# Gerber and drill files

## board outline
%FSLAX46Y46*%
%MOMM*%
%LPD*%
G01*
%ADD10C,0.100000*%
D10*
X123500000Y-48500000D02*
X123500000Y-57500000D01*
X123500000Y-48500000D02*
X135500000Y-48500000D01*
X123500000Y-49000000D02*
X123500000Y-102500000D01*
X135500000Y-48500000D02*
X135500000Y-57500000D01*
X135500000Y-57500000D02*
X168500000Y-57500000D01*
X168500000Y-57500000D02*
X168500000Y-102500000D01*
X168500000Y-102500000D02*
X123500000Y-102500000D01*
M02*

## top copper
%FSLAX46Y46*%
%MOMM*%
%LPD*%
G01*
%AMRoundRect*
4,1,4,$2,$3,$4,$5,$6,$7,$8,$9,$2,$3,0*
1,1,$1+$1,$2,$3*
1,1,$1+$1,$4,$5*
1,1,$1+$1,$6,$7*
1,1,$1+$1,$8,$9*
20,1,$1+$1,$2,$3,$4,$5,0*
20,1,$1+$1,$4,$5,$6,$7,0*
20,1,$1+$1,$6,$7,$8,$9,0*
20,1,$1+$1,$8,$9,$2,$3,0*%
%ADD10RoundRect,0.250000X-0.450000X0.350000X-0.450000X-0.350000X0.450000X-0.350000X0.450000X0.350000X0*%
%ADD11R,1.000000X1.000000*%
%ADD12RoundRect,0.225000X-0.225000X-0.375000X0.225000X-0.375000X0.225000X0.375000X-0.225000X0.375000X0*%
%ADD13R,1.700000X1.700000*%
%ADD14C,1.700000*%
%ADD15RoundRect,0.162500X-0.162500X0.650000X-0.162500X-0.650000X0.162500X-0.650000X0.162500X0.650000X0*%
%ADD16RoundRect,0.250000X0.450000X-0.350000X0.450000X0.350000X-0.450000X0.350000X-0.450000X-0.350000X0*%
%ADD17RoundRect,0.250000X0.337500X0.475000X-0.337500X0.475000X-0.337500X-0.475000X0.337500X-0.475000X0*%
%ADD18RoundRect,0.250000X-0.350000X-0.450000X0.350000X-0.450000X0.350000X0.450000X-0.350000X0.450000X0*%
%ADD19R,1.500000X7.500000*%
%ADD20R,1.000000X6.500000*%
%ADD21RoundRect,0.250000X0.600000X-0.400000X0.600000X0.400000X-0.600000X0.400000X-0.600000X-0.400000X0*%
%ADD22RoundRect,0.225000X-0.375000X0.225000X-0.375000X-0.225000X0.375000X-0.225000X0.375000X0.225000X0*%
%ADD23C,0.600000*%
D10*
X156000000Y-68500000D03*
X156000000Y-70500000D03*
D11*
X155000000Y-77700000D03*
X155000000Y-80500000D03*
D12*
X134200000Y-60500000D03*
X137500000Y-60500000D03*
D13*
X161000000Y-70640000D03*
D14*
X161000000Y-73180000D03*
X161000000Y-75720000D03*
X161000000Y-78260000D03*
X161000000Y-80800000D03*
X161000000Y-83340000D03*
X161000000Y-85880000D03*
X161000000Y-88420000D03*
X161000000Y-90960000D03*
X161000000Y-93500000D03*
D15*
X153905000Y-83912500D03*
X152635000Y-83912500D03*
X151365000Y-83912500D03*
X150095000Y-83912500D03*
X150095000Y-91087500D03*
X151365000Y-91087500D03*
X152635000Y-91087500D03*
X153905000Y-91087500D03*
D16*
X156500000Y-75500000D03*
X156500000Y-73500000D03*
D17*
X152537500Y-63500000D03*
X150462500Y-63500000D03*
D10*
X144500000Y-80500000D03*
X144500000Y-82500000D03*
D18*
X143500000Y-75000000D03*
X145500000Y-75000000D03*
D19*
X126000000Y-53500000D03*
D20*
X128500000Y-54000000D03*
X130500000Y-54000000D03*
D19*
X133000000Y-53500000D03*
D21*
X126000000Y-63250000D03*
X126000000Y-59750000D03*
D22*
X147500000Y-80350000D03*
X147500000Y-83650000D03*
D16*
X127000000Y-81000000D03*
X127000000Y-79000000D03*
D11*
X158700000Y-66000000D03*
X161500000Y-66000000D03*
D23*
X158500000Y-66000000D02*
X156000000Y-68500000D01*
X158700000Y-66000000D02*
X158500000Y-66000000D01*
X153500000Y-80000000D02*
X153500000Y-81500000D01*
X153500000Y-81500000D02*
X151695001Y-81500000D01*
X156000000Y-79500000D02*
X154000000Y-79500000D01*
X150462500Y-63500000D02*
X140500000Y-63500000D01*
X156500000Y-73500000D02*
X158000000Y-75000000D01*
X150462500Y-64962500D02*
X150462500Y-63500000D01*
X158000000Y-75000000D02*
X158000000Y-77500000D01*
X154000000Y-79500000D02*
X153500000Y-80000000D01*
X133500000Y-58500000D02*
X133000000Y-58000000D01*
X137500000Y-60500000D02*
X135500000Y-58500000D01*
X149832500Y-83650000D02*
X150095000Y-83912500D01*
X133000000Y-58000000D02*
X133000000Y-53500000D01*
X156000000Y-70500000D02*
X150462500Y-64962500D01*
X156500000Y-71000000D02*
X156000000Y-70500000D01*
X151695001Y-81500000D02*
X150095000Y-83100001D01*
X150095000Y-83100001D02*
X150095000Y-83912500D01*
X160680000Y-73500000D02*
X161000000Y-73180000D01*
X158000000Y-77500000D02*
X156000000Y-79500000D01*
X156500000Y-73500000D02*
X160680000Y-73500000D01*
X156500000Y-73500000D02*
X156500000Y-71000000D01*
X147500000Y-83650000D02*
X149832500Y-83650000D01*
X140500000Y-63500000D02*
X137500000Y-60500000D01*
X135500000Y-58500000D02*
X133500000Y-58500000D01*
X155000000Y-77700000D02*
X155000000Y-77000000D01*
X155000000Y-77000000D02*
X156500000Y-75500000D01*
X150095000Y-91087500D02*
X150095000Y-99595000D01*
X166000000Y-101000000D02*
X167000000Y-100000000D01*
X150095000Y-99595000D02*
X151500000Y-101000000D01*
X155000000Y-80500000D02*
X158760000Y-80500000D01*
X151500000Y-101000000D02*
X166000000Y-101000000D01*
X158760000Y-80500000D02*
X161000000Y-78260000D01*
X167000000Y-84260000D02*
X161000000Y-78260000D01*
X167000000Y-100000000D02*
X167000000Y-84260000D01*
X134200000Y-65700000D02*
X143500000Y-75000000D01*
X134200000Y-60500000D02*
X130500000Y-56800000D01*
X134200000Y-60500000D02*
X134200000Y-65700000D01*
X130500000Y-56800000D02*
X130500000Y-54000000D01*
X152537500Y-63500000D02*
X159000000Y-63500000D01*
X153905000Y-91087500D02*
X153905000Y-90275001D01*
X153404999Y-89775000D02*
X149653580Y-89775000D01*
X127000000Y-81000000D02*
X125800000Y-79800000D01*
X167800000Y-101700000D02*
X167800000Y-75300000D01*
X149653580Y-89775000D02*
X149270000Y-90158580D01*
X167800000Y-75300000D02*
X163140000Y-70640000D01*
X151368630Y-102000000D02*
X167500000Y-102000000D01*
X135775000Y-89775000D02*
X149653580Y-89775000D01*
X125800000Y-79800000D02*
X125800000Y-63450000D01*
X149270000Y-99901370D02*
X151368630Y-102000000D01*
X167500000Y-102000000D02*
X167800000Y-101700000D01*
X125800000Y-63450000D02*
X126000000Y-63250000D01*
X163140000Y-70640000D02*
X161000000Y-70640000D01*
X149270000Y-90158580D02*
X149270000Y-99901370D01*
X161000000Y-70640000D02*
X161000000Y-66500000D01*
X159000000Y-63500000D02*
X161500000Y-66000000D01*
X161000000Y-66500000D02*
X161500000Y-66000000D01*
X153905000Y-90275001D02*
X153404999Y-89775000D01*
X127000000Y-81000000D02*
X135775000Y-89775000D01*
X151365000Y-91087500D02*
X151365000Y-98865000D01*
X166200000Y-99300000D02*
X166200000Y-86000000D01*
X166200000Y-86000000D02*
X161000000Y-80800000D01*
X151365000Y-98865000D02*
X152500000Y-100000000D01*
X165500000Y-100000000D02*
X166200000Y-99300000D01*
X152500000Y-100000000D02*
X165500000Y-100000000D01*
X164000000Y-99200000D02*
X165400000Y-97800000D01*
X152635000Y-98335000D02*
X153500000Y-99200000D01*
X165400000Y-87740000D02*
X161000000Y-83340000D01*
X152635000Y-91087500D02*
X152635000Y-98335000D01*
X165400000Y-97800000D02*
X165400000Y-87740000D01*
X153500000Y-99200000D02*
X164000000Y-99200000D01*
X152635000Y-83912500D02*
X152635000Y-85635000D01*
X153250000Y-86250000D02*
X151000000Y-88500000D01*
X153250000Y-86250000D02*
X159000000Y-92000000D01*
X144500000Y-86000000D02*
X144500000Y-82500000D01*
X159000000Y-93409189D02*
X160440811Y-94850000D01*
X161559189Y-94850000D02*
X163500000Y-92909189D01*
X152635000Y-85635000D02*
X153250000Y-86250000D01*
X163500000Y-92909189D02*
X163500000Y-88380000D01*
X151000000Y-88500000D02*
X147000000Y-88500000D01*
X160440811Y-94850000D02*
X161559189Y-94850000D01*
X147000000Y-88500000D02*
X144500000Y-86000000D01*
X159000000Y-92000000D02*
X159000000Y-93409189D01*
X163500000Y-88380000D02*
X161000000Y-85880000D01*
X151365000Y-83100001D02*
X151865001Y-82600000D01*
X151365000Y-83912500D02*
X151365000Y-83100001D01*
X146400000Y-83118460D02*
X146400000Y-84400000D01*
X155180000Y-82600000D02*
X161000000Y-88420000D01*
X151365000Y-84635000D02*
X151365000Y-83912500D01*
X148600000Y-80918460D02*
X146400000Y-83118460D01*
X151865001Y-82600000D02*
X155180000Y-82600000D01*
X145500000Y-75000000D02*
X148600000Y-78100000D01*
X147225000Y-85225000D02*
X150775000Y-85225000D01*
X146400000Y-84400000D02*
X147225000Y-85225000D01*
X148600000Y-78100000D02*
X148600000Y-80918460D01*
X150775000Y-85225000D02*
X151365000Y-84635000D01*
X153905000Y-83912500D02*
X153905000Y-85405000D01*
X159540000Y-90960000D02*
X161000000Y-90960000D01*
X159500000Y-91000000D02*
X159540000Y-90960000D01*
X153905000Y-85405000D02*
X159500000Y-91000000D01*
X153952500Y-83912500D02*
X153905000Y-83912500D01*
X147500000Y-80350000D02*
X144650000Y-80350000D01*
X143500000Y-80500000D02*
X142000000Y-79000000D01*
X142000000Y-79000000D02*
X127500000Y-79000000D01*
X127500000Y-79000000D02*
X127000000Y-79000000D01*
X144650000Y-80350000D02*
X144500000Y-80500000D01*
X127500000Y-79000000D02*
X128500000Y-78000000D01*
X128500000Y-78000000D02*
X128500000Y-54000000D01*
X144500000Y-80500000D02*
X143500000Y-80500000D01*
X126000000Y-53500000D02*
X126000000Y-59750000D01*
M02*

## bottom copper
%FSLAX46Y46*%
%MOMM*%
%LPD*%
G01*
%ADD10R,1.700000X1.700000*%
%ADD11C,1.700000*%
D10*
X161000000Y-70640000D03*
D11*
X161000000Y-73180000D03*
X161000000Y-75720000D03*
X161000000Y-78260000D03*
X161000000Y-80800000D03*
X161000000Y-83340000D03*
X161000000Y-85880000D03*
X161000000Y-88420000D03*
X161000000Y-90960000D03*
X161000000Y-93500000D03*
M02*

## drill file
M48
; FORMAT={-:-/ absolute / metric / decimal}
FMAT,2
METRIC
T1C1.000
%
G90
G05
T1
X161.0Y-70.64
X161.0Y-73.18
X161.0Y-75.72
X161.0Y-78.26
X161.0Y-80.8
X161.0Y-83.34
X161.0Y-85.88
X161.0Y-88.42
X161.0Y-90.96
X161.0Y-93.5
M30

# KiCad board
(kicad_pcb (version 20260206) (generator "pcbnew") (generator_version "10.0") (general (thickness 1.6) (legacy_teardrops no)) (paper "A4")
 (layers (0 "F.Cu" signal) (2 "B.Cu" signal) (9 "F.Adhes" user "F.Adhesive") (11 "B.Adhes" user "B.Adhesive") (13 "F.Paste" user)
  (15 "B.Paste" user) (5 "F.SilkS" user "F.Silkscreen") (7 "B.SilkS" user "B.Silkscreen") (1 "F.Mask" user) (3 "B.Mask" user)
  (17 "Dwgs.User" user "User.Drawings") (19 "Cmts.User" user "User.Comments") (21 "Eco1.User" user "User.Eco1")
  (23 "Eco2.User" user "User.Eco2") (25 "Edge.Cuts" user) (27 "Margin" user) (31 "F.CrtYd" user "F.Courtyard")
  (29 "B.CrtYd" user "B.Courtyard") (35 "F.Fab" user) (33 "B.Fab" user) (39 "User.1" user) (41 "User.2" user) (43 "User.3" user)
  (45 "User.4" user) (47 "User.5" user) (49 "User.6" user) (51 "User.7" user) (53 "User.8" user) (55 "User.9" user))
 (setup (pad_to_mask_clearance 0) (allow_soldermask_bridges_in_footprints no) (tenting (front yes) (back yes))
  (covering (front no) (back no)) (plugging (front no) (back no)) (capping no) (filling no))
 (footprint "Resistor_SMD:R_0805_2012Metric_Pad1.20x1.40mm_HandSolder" (layer "F.Cu") (at 156 69.5 -90)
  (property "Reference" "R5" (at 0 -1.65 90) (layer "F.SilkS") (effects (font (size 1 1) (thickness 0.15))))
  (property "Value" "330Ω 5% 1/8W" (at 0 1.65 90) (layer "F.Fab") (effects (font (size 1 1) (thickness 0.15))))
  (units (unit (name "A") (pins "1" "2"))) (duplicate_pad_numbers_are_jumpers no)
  (pad "1" smd roundrect (at -1 0 270) (size 1.2 1.4) (layers "F.Cu" "F.Mask" "F.Paste") (roundrect_rratio 0.208333) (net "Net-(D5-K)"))
  (pad "2" smd roundrect (at 1 0 270) (size 1.2 1.4) (layers "F.Cu" "F.Mask" "F.Paste") (roundrect_rratio 0.208333) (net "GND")))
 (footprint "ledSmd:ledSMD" (layer "F.Cu") (at 155 79.5 -90)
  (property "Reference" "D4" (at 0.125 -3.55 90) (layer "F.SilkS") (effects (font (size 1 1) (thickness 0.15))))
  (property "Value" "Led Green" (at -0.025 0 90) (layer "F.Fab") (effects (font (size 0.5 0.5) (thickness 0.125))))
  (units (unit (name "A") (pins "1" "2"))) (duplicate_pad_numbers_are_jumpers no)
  (pad "1" smd rect (at -1.8 0 270) (size 1 1) (layers "F.Cu" "F.Mask" "F.Paste") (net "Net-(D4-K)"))
  (pad "2" smd rect (at 1 0 270) (size 1 1) (layers "F.Cu" "F.Mask" "F.Paste") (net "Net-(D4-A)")))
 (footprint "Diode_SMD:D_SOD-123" (layer "F.Cu") (at 135.85 60.5)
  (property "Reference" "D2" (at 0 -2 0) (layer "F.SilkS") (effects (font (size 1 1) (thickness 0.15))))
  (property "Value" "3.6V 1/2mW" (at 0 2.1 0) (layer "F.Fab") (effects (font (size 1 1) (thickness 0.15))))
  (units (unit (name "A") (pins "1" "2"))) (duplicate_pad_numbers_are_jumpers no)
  (pad "1" smd roundrect (at -1.65 0) (size 0.9 1.2) (layers "F.Cu" "F.Mask" "F.Paste") (roundrect_rratio 0.25) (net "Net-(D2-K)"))
  (pad "2" smd roundrect (at 1.65 0) (size 0.9 1.2) (layers "F.Cu" "F.Mask" "F.Paste") (roundrect_rratio 0.25) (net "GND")))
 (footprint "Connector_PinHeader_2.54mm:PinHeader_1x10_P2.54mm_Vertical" (layer "F.Cu") (at 161 70.64)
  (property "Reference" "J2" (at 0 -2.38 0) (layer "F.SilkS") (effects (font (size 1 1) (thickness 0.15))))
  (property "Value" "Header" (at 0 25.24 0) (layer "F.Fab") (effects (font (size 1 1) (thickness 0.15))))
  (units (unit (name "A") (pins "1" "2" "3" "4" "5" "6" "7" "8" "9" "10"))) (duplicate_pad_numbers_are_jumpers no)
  (pad "1" thru_hole rect (at 0 0) (size 1.7 1.7) (drill 1) (layers "*.Cu" "*.Mask") (remove_unused_layers no) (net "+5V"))
  (pad "2" thru_hole circle (at 0 2.54) (size 1.7 1.7) (drill 1) (layers "*.Cu" "*.Mask") (remove_unused_layers no) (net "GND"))
  (pad "3" thru_hole circle (at 0 5.08) (size 1.7 1.7) (drill 1) (layers "*.Cu" "*.Mask") (remove_unused_layers no)
   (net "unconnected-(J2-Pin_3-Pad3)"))
  (pad "4" thru_hole circle (at 0 7.62) (size 1.7 1.7) (drill 1) (layers "*.Cu" "*.Mask") (remove_unused_layers no) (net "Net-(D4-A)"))
  (pad "5" thru_hole circle (at 0 10.16) (size 1.7 1.7) (drill 1) (layers "*.Cu" "*.Mask") (remove_unused_layers no) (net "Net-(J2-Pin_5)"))
  (pad "6" thru_hole circle (at 0 12.7) (size 1.7 1.7) (drill 1) (layers "*.Cu" "*.Mask") (remove_unused_layers no) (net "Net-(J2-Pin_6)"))
  (pad "7" thru_hole circle (at 0 15.24) (size 1.7 1.7) (drill 1) (layers "*.Cu" "*.Mask") (remove_unused_layers no) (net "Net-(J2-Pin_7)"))
  (pad "8" thru_hole circle (at 0 17.78) (size 1.7 1.7) (drill 1) (layers "*.Cu" "*.Mask") (remove_unused_layers no) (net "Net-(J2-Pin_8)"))
  (pad "9" thru_hole circle (at 0 20.32) (size 1.7 1.7) (drill 1) (layers "*.Cu" "*.Mask") (remove_unused_layers no) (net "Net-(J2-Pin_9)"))
  (pad "10" thru_hole circle (at 0 22.86) (size 1.7 1.7) (drill 1) (layers "*.Cu" "*.Mask") (remove_unused_layers no)
   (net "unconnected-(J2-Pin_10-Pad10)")))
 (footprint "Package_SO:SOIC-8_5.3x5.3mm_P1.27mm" (layer "F.Cu") (at 152 87.5 -90)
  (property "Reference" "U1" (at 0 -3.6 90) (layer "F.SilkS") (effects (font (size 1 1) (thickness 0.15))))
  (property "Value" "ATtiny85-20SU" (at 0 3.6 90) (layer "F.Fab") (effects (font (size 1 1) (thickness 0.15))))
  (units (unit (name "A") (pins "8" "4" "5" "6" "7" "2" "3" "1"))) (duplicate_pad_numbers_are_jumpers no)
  (pad "1" smd roundrect (at -3.5875 -1.905 270) (size 1.625 0.65) (layers "F.Cu" "F.Mask" "F.Paste") (roundrect_rratio 0.25)
   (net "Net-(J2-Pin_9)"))
  (pad "2" smd roundrect (at -3.5875 -0.635 270) (size 1.625 0.65) (layers "F.Cu" "F.Mask" "F.Paste") (roundrect_rratio 0.25)
   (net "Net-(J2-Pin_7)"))
  (pad "3" smd roundrect (at -3.5875 0.635 270) (size 1.625 0.65) (layers "F.Cu" "F.Mask" "F.Paste") (roundrect_rratio 0.25)
   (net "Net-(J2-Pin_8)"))
  (pad "4" smd roundrect (at -3.5875 1.905 270) (size 1.625 0.65) (layers "F.Cu" "F.Mask" "F.Paste") (roundrect_rratio 0.25) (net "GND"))
  (pad "5" smd roundrect (at 3.5875 1.905 270) (size 1.625 0.65) (layers "F.Cu" "F.Mask" "F.Paste") (roundrect_rratio 0.25)
   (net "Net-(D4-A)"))
  (pad "6" smd roundrect (at 3.5875 0.635 270) (size 1.625 0.65) (layers "F.Cu" "F.Mask" "F.Paste") (roundrect_rratio 0.25)
   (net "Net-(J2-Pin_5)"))
  (pad "7" smd roundrect (at 3.5875 -0.635 270) (size 1.625 0.65) (layers "F.Cu" "F.Mask" "F.Paste") (roundrect_rratio 0.25)
   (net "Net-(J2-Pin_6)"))
  (pad "8" smd roundrect (at 3.5875 -1.905 270) (size 1.625 0.65) (layers "F.Cu" "F.Mask" "F.Paste") (roundrect_rratio 0.25) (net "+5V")))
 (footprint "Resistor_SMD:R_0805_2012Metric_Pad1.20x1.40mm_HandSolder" (layer "F.Cu") (at 156.5 74.5 90)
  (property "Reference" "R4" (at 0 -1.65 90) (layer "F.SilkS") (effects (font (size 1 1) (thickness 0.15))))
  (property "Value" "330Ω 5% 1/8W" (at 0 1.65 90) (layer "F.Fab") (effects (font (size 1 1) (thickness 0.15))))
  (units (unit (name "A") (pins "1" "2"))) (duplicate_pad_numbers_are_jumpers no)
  (pad "1" smd roundrect (at -1 0 90) (size 1.2 1.4) (layers "F.Cu" "F.Mask" "F.Paste") (roundrect_rratio 0.208333) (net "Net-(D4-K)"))
  (pad "2" smd roundrect (at 1 0 90) (size 1.2 1.4) (layers "F.Cu" "F.Mask" "F.Paste") (roundrect_rratio 0.208333) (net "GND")))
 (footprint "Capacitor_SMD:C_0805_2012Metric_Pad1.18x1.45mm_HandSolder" (layer "F.Cu") (at 151.5 63.5 180)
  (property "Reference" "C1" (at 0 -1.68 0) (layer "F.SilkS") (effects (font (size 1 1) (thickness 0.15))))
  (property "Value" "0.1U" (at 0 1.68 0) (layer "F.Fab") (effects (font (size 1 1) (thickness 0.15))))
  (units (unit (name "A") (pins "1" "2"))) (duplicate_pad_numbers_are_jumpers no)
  (pad "1" smd roundrect (at -1.0375 0 180) (size 1.175 1.45) (layers "F.Cu" "F.Mask" "F.Paste") (roundrect_rratio 0.212766) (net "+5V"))
  (pad "2" smd roundrect (at 1.0375 0 180) (size 1.175 1.45) (layers "F.Cu" "F.Mask" "F.Paste") (roundrect_rratio 0.212766) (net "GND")))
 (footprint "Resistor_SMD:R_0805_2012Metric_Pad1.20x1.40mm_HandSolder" (layer "F.Cu") (at 144.5 81.5 -90)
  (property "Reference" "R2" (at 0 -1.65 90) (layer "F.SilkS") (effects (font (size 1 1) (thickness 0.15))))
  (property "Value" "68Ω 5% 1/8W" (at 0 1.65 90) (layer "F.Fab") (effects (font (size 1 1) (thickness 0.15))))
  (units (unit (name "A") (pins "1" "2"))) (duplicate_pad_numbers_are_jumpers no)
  (pad "1" smd roundrect (at -1 0 270) (size 1.2 1.4) (layers "F.Cu" "F.Mask" "F.Paste") (roundrect_rratio 0.208333) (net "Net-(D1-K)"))
  (pad "2" smd roundrect (at 1 0 270) (size 1.2 1.4) (layers "F.Cu" "F.Mask" "F.Paste") (roundrect_rratio 0.208333) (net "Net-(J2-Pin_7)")))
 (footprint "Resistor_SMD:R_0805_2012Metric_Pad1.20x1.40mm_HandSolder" (layer "F.Cu") (at 144.5 75)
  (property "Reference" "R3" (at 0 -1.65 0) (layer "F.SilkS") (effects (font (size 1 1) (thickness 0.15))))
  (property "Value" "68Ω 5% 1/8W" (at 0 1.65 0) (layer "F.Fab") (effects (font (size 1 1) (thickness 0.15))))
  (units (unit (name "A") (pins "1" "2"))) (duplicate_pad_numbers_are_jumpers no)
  (pad "1" smd roundrect (at -1 0) (size 1.2 1.4) (layers "F.Cu" "F.Mask" "F.Paste") (roundrect_rratio 0.208333) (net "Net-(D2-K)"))
  (pad "2" smd roundrect (at 1 0) (size 1.2 1.4) (layers "F.Cu" "F.Mask" "F.Paste") (roundrect_rratio 0.208333) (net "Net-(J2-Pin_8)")))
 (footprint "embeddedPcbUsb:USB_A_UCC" (layer "F.Cu") (at 129.5 53.7 -90)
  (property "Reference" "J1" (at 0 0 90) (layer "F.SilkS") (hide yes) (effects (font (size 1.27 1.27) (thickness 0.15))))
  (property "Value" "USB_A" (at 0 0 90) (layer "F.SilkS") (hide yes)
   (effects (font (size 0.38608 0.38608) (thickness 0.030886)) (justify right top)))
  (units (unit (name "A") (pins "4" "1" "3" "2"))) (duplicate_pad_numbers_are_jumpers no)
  (pad "1" smd rect (at -0.2 3.5 270) (size 7.5 1.5) (layers "F.Cu" "F.Mask" "F.Paste") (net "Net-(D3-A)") (solder_mask_margin 0.1016))
  (pad "2" smd rect (at 0.3 1 270) (size 6.5 1) (layers "F.Cu" "F.Mask" "F.Paste") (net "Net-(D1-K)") (solder_mask_margin 0.1016))
  (pad "3" smd rect (at 0.3 -1 270) (size 6.5 1) (layers "F.Cu" "F.Mask" "F.Paste") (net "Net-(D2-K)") (solder_mask_margin 0.1016))
  (pad "4" smd rect (at -0.2 -3.5 270) (size 7.5 1.5) (layers "F.Cu" "F.Mask" "F.Paste") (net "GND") (solder_mask_margin 0.1016)))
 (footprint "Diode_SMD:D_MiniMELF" (layer "F.Cu") (at 126 61.5 90)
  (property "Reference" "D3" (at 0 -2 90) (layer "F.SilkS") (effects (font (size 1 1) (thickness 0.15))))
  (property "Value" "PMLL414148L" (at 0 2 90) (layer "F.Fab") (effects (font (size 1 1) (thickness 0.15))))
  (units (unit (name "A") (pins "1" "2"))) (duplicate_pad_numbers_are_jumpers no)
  (pad "1" smd roundrect (at -1.75 0 90) (size 1.3 1.7) (layers "F.Cu" "F.Mask" "F.Paste") (roundrect_rratio 0.1923076923) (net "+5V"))
  (pad "2" smd roundrect (at 1.75 0 90) (size 1.3 1.7) (layers "F.Cu" "F.Mask" "F.Paste") (roundrect_rratio 0.1923076923) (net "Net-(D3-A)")))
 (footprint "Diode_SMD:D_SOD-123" (layer "F.Cu") (at 147.5 82 -90)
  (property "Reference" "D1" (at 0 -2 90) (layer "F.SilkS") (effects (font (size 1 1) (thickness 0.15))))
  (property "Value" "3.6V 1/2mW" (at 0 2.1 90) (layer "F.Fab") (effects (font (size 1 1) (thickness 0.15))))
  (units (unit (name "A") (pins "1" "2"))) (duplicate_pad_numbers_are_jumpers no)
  (pad "1" smd roundrect (at -1.65 0 270) (size 0.9 1.2) (layers "F.Cu" "F.Mask" "F.Paste") (roundrect_rratio 0.25) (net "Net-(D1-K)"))
  (pad "2" smd roundrect (at 1.65 0 270) (size 0.9 1.2) (layers "F.Cu" "F.Mask" "F.Paste") (roundrect_rratio 0.25) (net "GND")))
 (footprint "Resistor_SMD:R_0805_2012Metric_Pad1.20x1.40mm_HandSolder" (layer "F.Cu") (at 127 80 90)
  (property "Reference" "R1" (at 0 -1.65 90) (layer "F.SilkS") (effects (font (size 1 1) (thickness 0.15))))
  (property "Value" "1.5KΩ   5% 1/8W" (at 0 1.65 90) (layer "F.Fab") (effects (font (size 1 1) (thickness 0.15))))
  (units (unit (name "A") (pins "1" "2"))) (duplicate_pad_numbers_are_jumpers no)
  (pad "1" smd roundrect (at -1 0 90) (size 1.2 1.4) (layers "F.Cu" "F.Mask" "F.Paste") (roundrect_rratio 0.208333) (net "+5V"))
  (pad "2" smd roundrect (at 1 0 90) (size 1.2 1.4) (layers "F.Cu" "F.Mask" "F.Paste") (roundrect_rratio 0.208333) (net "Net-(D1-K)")))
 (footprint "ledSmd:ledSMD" (layer "F.Cu") (at 160.5 66)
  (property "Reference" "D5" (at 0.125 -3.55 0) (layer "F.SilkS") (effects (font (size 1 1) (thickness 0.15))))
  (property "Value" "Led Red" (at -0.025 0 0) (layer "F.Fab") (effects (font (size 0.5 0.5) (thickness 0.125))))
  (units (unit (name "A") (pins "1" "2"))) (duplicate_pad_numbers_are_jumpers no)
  (pad "1" smd rect (at -1.8 0) (size 1 1) (layers "F.Cu" "F.Mask" "F.Paste") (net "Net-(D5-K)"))
  (pad "2" smd rect (at 1 0) (size 1 1) (layers "F.Cu" "F.Mask" "F.Paste") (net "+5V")))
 (gr_line (start 123.5 48.5) (end 123.5 57.5) (stroke (width 0.1) (type default)) (layer "Edge.Cuts"))
 (gr_line (start 123.5 48.5) (end 135.5 48.5) (stroke (width 0.1) (type default)) (layer "Edge.Cuts"))
 (gr_line (start 123.5 49) (end 123.5 102.5) (stroke (width 0.1) (type default)) (layer "Edge.Cuts"))
 (gr_line (start 135.5 48.5) (end 135.5 57.5) (stroke (width 0.1) (type default)) (layer "Edge.Cuts"))
 (gr_line (start 135.5 57.5) (end 168.5 57.5) (stroke (width 0.1) (type default)) (layer "Edge.Cuts"))
 (gr_line (start 168.5 57.5) (end 168.5 102.5) (stroke (width 0.1) (type default)) (layer "Edge.Cuts"))
 (gr_line (start 168.5 102.5) (end 123.5 102.5) (stroke (width 0.1) (type default)) (layer "Edge.Cuts"))
 (segment (start 158.5 66) (end 156 68.5) (width 0.6) (layer "F.Cu") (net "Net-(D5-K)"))
 (segment (start 158.7 66) (end 158.5 66) (width 0.6) (layer "F.Cu") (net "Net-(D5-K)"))
 (segment (start 153.5 80) (end 153.5 81.5) (width 0.6) (layer "F.Cu") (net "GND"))
 (segment (start 153.5 81.5) (end 151.695001 81.5) (width 0.6) (layer "F.Cu") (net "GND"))
 (segment (start 156 79.5) (end 154 79.5) (width 0.6) (layer "F.Cu") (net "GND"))
 (segment (start 150.4625 63.5) (end 140.5 63.5) (width 0.6) (layer "F.Cu") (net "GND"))
 (segment (start 156.5 73.5) (end 158 75) (width 0.6) (layer "F.Cu") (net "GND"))
 (segment (start 150.4625 64.9625) (end 150.4625 63.5) (width 0.6) (layer "F.Cu") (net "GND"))
 (segment (start 158 75) (end 158 77.5) (width 0.6) (layer "F.Cu") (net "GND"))
 (segment (start 154 79.5) (end 153.5 80) (width 0.6) (layer "F.Cu") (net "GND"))
 (segment (start 133.5 58.5) (end 133 58) (width 0.6) (layer "F.Cu") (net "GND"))
 (segment (start 137.5 60.5) (end 135.5 58.5) (width 0.6) (layer "F.Cu") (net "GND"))
 (segment (start 149.8325 83.65) (end 150.095 83.9125) (width 0.6) (layer "F.Cu") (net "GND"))
 (segment (start 133 58) (end 133 53.5) (width 0.6) (layer "F.Cu") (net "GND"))
 (segment (start 156 70.5) (end 150.4625 64.9625) (width 0.6) (layer "F.Cu") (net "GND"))
 (segment (start 156.5 71) (end 156 70.5) (width 0.6) (layer "F.Cu") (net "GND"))
 (segment (start 151.695001 81.5) (end 150.095 83.100001) (width 0.6) (layer "F.Cu") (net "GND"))
 (segment (start 150.095 83.100001) (end 150.095 83.9125) (width 0.6) (layer "F.Cu") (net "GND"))
 (segment (start 160.68 73.5) (end 161 73.18) (width 0.6) (layer "F.Cu") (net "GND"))
 (segment (start 158 77.5) (end 156 79.5) (width 0.6) (layer "F.Cu") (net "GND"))
 (segment (start 156.5 73.5) (end 160.68 73.5) (width 0.6) (layer "F.Cu") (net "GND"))
 (segment (start 156.5 73.5) (end 156.5 71) (width 0.6) (layer "F.Cu") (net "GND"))
 (segment (start 147.5 83.65) (end 149.8325 83.65) (width 0.6) (layer "F.Cu") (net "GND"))
 (segment (start 140.5 63.5) (end 137.5 60.5) (width 0.6) (layer "F.Cu") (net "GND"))
 (segment (start 135.5 58.5) (end 133.5 58.5) (width 0.6) (layer "F.Cu") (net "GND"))
 (segment (start 155 77.7) (end 155 77) (width 0.6) (layer "F.Cu") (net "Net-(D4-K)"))
 (segment (start 155 77) (end 156.5 75.5) (width 0.6) (layer "F.Cu") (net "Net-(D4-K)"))
 (segment (start 150.095 91.0875) (end 150.095 99.595) (width 0.6) (layer "F.Cu") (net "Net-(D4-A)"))
 (segment (start 166 101) (end 167 100) (width 0.6) (layer "F.Cu") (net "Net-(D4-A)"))
 (segment (start 150.095 99.595) (end 151.5 101) (width 0.6) (layer "F.Cu") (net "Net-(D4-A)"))
 (segment (start 155 80.5) (end 158.76 80.5) (width 0.6) (layer "F.Cu") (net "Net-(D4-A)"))
 (segment (start 151.5 101) (end 166 101) (width 0.6) (layer "F.Cu") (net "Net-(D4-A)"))
 (segment (start 158.76 80.5) (end 161 78.26) (width 0.6) (layer "F.Cu") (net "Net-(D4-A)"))
 (segment (start 167 84.26) (end 161 78.26) (width 0.6) (layer "F.Cu") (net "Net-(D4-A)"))
 (segment (start 167 100) (end 167 84.26) (width 0.6) (layer "F.Cu") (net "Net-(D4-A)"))
 (segment (start 134.2 65.7) (end 143.5 75) (width 0.6) (layer "F.Cu") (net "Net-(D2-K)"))
 (segment (start 134.2 60.5) (end 130.5 56.8) (width 0.6) (layer "F.Cu") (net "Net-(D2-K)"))
 (segment (start 134.2 60.5) (end 134.2 65.7) (width 0.6) (layer "F.Cu") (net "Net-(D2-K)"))
 (segment (start 130.5 56.8) (end 130.5 54) (width 0.6) (layer "F.Cu") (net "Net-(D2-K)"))
 (segment (start 152.5375 63.5) (end 159 63.5) (width 0.6) (layer "F.Cu") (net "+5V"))
 (segment (start 153.905 91.0875) (end 153.905 90.275001) (width 0.6) (layer "F.Cu") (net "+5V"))
 (segment (start 153.404999 89.775) (end 149.65358 89.775) (width 0.6) (layer "F.Cu") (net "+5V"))
 (segment (start 127 81) (end 125.8 79.8) (width 0.6) (layer "F.Cu") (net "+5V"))
 (segment (start 167.8 101.7) (end 167.8 75.3) (width 0.6) (layer "F.Cu") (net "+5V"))
 (segment (start 149.65358 89.775) (end 149.27 90.15858) (width 0.6) (layer "F.Cu") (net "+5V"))
 (segment (start 167.8 75.3) (end 163.14 70.64) (width 0.6) (layer "F.Cu") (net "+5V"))
 (segment (start 151.36863 102) (end 167.5 102) (width 0.6) (layer "F.Cu") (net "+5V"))
 (segment (start 135.775 89.775) (end 149.65358 89.775) (width 0.6) (layer "F.Cu") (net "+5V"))
 (segment (start 125.8 79.8) (end 125.8 63.45) (width 0.6) (layer "F.Cu") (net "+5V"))
 (segment (start 149.27 99.90137) (end 151.36863 102) (width 0.6) (layer "F.Cu") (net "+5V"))
 (segment (start 167.5 102) (end 167.8 101.7) (width 0.6) (layer "F.Cu") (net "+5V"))
 (segment (start 125.8 63.45) (end 126 63.25) (width 0.6) (layer "F.Cu") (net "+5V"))
 (segment (start 163.14 70.64) (end 161 70.64) (width 0.6) (layer "F.Cu") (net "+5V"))
 (segment (start 149.27 90.15858) (end 149.27 99.90137) (width 0.6) (layer "F.Cu") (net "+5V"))
 (segment (start 161 70.64) (end 161 66.5) (width 0.6) (layer "F.Cu") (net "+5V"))
 (segment (start 159 63.5) (end 161.5 66) (width 0.6) (layer "F.Cu") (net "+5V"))
 (segment (start 161 66.5) (end 161.5 66) (width 0.6) (layer "F.Cu") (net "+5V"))
 (segment (start 153.905 90.275001) (end 153.404999 89.775) (width 0.6) (layer "F.Cu") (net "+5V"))
 (segment (start 127 81) (end 135.775 89.775) (width 0.6) (layer "F.Cu") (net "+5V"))
 (segment (start 151.365 91.0875) (end 151.365 98.865) (width 0.6) (layer "F.Cu") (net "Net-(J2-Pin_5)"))
 (segment (start 166.2 99.3) (end 166.2 86) (width 0.6) (layer "F.Cu") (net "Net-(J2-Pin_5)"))
 (segment (start 166.2 86) (end 161 80.8) (width 0.6) (layer "F.Cu") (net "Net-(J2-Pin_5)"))
 (segment (start 151.365 98.865) (end 152.5 100) (width 0.6) (layer "F.Cu") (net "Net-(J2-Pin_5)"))
 (segment (start 165.5 100) (end 166.2 99.3) (width 0.6) (layer "F.Cu") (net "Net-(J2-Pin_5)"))
 (segment (start 152.5 100) (end 165.5 100) (width 0.6) (layer "F.Cu") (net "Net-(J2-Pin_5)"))
 (segment (start 164 99.2) (end 165.4 97.8) (width 0.6) (layer "F.Cu") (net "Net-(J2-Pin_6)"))
 (segment (start 152.635 98.335) (end 153.5 99.2) (width 0.6) (layer "F.Cu") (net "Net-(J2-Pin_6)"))
 (segment (start 165.4 87.74) (end 161 83.34) (width 0.6) (layer "F.Cu") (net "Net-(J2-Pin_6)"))
 (segment (start 152.635 91.0875) (end 152.635 98.335) (width 0.6) (layer "F.Cu") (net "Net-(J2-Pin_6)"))
 (segment (start 165.4 97.8) (end 165.4 87.74) (width 0.6) (layer "F.Cu") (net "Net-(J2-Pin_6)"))
 (segment (start 153.5 99.2) (end 164 99.2) (width 0.6) (layer "F.Cu") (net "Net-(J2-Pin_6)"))
 (segment (start 152.635 83.9125) (end 152.635 85.635) (width 0.6) (layer "F.Cu") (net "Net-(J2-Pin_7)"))
 (segment (start 153.25 86.25) (end 151 88.5) (width 0.6) (layer "F.Cu") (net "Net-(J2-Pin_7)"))
 (segment (start 153.25 86.25) (end 159 92) (width 0.6) (layer "F.Cu") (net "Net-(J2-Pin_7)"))
 (segment (start 144.5 86) (end 144.5 82.5) (width 0.6) (layer "F.Cu") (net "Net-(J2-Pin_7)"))
 (segment (start 159 93.409189) (end 160.440811 94.85) (width 0.6) (layer "F.Cu") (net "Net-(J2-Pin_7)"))
 (segment (start 161.559189 94.85) (end 163.5 92.909189) (width 0.6) (layer "F.Cu") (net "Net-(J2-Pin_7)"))
 (segment (start 152.635 85.635) (end 153.25 86.25) (width 0.6) (layer "F.Cu") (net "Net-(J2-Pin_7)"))
 (segment (start 163.5 92.909189) (end 163.5 88.38) (width 0.6) (layer "F.Cu") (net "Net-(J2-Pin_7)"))
 (segment (start 151 88.5) (end 147 88.5) (width 0.6) (layer "F.Cu") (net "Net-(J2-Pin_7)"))
 (segment (start 160.440811 94.85) (end 161.559189 94.85) (width 0.6) (layer "F.Cu") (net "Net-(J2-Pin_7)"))
 (segment (start 147 88.5) (end 144.5 86) (width 0.6) (layer "F.Cu") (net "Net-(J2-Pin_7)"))
 (segment (start 159 92) (end 159 93.409189) (width 0.6) (layer "F.Cu") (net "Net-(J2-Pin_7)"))
 (segment (start 163.5 88.38) (end 161 85.88) (width 0.6) (layer "F.Cu") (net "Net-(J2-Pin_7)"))
 (segment (start 151.365 83.100001) (end 151.865001 82.6) (width 0.6) (layer "F.Cu") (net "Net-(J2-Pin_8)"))
 (segment (start 151.365 83.9125) (end 151.365 83.100001) (width 0.6) (layer "F.Cu") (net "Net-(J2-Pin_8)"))
 (segment (start 146.4 83.11846) (end 146.4 84.4) (width 0.6) (layer "F.Cu") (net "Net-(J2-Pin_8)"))
 (segment (start 155.18 82.6) (end 161 88.42) (width 0.6) (layer "F.Cu") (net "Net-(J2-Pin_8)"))
 (segment (start 151.365 84.635) (end 151.365 83.9125) (width 0.6) (layer "F.Cu") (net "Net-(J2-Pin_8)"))
 (segment (start 148.6 80.91846) (end 146.4 83.11846) (width 0.6) (layer "F.Cu") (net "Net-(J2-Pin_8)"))
 (segment (start 151.865001 82.6) (end 155.18 82.6) (width 0.6) (layer "F.Cu") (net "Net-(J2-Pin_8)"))
 (segment (start 145.5 75) (end 148.6 78.1) (width 0.6) (layer "F.Cu") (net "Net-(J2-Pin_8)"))
 (segment (start 147.225 85.225) (end 150.775 85.225) (width 0.6) (layer "F.Cu") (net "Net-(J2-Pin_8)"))
 (segment (start 146.4 84.4) (end 147.225 85.225) (width 0.6) (layer "F.Cu") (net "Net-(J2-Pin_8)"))
 (segment (start 148.6 78.1) (end 148.6 80.91846) (width 0.6) (layer "F.Cu") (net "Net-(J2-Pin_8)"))
 (segment (start 150.775 85.225) (end 151.365 84.635) (width 0.6) (layer "F.Cu") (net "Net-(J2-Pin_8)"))
 (segment (start 153.905 83.9125) (end 153.905 85.405) (width 0.6) (layer "F.Cu") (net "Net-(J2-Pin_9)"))
 (segment (start 159.54 90.96) (end 161 90.96) (width 0.6) (layer "F.Cu") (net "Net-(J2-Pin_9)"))
 (segment (start 159.5 91) (end 159.54 90.96) (width 0.6) (layer "F.Cu") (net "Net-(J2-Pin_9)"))
 (segment (start 153.905 85.405) (end 159.5 91) (width 0.6) (layer "F.Cu") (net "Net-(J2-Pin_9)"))
 (segment (start 153.9525 83.9125) (end 153.905 83.9125) (width 0.6) (layer "F.Cu") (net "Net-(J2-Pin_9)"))
 (segment (start 147.5 80.35) (end 144.65 80.35) (width 0.6) (layer "F.Cu") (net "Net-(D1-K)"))
 (segment (start 143.5 80.5) (end 142 79) (width 0.6) (layer "F.Cu") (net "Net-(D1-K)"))
 (segment (start 142 79) (end 127.5 79) (width 0.6) (layer "F.Cu") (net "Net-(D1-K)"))
 (segment (start 127.5 79) (end 127 79) (width 0.6) (layer "F.Cu") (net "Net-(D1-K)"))
 (segment (start 144.65 80.35) (end 144.5 80.5) (width 0.6) (layer "F.Cu") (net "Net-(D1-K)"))
 (segment (start 127.5 79) (end 128.5 78) (width 0.6) (layer "F.Cu") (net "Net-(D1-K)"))
 (segment (start 128.5 78) (end 128.5 54) (width 0.6) (layer "F.Cu") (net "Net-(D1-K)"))
 (segment (start 144.5 80.5) (end 143.5 80.5) (width 0.6) (layer "F.Cu") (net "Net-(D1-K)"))
 (segment (start 126 53.5) (end 126 59.75) (width 0.6) (layer "F.Cu") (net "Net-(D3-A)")))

